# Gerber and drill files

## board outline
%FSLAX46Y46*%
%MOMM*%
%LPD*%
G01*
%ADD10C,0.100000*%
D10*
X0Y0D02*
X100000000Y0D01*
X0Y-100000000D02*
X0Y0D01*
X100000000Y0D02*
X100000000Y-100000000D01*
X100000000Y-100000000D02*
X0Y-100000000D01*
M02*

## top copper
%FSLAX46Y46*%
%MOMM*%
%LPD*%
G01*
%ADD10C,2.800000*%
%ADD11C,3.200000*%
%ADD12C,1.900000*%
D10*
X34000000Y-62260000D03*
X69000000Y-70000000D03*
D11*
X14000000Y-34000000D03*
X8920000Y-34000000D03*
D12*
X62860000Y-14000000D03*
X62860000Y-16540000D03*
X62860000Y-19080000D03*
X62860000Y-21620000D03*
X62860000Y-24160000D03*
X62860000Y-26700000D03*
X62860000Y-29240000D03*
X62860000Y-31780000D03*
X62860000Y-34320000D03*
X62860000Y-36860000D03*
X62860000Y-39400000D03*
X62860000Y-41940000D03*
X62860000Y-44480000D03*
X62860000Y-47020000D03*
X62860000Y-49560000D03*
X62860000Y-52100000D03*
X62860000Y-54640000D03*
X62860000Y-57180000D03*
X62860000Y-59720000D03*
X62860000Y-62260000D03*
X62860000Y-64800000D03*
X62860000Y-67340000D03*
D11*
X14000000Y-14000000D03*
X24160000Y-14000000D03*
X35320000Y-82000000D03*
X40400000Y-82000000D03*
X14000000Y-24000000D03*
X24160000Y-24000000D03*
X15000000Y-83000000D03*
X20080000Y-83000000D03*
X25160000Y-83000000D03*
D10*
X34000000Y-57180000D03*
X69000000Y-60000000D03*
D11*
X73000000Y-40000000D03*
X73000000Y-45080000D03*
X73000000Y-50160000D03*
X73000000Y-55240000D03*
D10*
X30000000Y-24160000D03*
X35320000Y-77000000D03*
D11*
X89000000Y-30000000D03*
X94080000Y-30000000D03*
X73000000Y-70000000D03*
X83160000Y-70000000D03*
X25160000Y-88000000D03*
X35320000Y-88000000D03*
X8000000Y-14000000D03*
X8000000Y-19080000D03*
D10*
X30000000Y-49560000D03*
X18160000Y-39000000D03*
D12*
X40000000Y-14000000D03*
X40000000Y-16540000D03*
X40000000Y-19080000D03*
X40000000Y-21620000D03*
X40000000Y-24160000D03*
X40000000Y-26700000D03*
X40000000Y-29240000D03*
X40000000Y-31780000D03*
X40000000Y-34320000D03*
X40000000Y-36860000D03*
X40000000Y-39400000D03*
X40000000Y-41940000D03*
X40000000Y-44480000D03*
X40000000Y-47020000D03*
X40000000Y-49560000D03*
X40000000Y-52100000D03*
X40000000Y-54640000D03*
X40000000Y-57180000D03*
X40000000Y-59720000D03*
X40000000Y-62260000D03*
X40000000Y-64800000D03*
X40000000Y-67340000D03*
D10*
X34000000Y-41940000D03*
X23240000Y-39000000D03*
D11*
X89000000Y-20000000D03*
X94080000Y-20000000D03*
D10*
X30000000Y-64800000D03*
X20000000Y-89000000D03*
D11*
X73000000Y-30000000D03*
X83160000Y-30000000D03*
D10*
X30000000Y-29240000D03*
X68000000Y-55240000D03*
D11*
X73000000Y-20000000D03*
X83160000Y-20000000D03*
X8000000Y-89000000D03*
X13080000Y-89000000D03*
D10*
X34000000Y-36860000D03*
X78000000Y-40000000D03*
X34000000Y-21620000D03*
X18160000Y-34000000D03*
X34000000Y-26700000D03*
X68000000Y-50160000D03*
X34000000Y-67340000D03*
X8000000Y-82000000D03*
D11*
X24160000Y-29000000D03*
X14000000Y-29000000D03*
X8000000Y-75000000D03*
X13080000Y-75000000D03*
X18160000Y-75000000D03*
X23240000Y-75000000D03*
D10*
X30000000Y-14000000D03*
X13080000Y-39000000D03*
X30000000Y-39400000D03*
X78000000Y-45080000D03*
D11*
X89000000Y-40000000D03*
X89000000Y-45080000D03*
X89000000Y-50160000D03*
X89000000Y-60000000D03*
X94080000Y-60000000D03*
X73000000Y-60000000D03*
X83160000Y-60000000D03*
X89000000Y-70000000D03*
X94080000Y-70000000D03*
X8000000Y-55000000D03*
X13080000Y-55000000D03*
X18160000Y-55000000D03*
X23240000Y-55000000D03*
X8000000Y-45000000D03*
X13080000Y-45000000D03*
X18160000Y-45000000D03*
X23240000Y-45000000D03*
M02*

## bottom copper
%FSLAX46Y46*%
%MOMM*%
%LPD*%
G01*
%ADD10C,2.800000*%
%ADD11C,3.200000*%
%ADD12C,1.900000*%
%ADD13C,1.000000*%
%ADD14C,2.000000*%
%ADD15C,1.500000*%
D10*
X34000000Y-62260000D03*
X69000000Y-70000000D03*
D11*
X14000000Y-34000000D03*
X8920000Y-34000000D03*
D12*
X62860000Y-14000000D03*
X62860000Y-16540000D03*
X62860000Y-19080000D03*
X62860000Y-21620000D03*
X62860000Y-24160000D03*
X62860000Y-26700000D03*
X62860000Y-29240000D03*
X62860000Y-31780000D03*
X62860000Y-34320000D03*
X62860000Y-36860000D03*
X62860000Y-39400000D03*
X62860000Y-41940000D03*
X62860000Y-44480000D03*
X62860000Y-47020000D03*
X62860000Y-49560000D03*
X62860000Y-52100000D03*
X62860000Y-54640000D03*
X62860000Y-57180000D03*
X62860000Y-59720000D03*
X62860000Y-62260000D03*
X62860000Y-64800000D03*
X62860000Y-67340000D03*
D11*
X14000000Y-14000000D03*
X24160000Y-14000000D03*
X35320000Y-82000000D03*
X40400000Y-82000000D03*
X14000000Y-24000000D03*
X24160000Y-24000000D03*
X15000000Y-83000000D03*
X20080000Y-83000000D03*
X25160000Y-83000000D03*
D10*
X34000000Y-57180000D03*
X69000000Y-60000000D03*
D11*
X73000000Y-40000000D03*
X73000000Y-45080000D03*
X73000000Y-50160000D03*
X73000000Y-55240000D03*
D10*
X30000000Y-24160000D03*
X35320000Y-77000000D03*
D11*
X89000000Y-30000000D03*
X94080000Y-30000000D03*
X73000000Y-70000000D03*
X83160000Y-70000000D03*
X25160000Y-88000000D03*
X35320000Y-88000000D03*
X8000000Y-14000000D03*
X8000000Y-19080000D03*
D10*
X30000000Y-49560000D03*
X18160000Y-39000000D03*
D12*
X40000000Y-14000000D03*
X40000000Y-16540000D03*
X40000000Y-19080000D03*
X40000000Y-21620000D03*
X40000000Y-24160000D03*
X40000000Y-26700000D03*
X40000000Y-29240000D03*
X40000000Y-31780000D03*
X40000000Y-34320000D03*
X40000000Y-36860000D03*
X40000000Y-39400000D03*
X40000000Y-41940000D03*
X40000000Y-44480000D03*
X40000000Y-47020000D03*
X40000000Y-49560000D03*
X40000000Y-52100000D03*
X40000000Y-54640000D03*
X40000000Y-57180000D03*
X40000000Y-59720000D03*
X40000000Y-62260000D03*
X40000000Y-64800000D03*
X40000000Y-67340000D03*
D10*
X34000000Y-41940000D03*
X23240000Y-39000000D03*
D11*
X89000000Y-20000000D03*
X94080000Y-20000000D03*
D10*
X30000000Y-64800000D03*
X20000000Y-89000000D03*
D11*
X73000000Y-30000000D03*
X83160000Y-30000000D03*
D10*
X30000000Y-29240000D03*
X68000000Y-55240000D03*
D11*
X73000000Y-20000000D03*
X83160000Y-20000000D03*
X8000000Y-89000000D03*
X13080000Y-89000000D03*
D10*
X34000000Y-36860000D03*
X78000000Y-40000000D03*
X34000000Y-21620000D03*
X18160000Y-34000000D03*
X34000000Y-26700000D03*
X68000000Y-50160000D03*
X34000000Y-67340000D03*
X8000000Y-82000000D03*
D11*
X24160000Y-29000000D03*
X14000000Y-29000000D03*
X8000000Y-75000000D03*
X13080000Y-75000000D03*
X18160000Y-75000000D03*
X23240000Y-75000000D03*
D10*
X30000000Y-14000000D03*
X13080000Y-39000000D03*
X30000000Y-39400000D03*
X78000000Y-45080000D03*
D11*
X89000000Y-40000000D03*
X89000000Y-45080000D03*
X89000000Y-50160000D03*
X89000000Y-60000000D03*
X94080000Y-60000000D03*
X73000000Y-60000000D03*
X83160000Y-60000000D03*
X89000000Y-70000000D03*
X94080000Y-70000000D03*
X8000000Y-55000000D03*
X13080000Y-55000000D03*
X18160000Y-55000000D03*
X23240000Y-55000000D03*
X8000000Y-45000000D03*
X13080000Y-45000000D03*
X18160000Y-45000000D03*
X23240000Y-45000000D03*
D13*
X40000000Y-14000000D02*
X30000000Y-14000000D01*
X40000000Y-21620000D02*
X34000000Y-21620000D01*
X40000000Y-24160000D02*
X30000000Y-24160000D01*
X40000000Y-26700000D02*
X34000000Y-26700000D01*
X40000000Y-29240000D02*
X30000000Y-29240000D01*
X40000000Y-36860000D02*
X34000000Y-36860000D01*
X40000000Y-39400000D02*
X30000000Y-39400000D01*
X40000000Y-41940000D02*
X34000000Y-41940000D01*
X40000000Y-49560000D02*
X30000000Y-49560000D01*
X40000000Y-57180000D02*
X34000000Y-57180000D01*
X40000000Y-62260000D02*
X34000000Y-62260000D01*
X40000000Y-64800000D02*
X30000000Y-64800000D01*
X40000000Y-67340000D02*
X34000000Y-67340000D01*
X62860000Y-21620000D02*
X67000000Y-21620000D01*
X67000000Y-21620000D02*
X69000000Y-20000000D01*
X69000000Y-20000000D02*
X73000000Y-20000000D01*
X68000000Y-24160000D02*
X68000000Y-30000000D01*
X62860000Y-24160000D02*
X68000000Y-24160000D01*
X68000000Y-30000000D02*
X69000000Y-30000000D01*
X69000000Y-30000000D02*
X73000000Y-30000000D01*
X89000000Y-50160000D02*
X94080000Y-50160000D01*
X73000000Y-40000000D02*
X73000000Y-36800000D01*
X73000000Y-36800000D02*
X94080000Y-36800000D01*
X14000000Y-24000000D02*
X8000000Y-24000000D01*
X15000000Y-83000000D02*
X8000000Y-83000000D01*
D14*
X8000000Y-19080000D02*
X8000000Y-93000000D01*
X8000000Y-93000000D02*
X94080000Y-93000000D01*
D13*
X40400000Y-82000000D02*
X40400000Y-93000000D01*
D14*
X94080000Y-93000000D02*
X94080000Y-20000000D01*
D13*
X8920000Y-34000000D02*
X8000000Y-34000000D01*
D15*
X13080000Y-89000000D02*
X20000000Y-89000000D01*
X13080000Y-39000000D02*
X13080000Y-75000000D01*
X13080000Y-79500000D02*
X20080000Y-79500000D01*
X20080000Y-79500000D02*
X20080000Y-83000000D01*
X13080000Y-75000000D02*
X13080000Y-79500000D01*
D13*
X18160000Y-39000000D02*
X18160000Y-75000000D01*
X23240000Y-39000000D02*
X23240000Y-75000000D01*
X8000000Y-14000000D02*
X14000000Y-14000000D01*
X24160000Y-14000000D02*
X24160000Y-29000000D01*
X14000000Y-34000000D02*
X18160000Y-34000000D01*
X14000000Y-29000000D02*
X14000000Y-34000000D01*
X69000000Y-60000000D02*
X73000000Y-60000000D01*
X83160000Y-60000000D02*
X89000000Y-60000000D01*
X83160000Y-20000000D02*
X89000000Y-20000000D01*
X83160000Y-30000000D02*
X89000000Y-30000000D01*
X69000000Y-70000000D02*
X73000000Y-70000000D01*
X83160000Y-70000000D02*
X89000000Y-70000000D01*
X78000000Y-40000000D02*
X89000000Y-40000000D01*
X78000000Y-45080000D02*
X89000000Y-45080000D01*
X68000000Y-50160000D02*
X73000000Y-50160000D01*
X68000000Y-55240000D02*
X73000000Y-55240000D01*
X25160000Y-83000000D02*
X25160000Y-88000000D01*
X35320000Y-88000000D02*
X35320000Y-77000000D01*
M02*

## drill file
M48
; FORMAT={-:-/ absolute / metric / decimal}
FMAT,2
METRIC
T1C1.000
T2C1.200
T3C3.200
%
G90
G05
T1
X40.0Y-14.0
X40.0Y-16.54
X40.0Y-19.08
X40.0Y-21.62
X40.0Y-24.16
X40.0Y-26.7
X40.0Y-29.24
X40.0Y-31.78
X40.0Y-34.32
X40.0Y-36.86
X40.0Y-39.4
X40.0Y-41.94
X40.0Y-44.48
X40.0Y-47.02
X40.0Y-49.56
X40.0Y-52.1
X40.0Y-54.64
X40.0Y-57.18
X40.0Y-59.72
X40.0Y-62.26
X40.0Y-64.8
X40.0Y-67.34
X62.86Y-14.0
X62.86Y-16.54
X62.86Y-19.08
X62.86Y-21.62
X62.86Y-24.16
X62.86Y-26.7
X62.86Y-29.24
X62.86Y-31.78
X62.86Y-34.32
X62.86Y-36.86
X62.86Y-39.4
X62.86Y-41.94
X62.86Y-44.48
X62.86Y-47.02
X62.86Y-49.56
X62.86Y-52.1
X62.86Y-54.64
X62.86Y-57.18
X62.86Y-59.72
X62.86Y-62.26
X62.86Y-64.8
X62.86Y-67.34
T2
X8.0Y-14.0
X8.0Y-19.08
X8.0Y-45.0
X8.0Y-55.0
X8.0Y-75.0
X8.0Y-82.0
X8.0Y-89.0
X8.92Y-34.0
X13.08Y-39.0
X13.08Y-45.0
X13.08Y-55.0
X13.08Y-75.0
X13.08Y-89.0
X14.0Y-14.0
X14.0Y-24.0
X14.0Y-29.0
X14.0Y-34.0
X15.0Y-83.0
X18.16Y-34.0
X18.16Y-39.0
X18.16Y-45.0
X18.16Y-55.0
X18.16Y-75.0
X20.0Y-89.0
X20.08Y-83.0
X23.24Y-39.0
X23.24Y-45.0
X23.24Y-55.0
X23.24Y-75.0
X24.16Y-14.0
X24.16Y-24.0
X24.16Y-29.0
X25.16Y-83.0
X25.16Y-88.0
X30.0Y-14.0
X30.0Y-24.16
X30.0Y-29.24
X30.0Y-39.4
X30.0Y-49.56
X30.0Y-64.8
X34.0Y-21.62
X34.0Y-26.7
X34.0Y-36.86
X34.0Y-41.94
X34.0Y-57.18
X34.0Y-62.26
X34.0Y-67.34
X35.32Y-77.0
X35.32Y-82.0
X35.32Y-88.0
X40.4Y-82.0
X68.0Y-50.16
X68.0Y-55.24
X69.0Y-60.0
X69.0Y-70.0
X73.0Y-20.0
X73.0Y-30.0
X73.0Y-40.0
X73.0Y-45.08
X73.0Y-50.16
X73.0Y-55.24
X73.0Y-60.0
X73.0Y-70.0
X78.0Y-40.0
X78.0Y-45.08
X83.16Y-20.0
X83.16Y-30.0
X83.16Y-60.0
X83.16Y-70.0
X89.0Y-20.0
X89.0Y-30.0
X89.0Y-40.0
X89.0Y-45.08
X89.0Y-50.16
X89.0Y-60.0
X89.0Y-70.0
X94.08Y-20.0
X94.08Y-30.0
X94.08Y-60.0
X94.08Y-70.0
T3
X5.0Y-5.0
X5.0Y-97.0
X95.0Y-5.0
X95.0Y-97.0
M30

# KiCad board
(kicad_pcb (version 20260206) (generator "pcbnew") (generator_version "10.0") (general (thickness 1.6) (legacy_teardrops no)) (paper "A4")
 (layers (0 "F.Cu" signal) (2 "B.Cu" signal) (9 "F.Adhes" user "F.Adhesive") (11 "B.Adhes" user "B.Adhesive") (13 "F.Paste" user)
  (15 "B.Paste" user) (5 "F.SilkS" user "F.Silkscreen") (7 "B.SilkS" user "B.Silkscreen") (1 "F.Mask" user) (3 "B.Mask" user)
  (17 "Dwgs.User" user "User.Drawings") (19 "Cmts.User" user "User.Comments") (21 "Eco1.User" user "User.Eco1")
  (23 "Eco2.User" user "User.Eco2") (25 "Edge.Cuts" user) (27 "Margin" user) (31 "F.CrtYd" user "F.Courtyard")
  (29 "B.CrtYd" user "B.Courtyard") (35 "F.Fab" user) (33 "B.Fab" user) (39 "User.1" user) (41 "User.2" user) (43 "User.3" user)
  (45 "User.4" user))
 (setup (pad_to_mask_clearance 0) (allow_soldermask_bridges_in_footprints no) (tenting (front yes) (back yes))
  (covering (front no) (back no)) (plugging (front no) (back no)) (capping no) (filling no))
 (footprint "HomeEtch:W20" (layer "F.Cu") (at 34 62.26)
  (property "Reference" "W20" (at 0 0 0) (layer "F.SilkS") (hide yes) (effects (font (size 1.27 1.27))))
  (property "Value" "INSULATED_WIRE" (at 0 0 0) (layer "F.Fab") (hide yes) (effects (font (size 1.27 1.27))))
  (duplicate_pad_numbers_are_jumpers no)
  (pad "1" thru_hole circle (at 0 0) (size 2.8 2.8) (drill 1.2) (layers "*.Cu" "*.Mask") (remove_unused_layers no) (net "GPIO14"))
  (pad "2" thru_hole circle (at 35 7.74) (size 2.8 2.8) (drill 1.2) (layers "*.Cu" "*.Mask") (remove_unused_layers no) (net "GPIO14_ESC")))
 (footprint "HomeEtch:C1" (layer "F.Cu") (at 14 34)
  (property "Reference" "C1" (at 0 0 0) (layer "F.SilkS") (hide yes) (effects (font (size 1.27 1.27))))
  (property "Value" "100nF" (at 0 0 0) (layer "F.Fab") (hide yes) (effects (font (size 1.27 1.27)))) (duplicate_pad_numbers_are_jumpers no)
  (pad "1" thru_hole circle (at 0 0) (size 3.2 3.2) (drill 1.2) (layers "*.Cu" "*.Mask") (remove_unused_layers no) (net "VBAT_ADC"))
  (pad "2" thru_hole circle (at -5.08 0) (size 3.2 3.2) (drill 1.2) (layers "*.Cu" "*.Mask") (remove_unused_layers no) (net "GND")))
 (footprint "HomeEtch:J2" (layer "F.Cu") (at 62.86 14)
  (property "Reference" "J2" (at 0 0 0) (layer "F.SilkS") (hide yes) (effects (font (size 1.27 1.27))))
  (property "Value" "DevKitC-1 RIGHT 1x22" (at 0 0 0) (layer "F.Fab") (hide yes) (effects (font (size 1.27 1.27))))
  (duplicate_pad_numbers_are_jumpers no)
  (pad "1" thru_hole circle (at 0 0) (size 1.9 1.9) (drill 1) (layers "*.Cu" "*.Mask") (remove_unused_layers no)
   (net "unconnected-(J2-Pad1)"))
  (pad "2" thru_hole circle (at 0 2.54) (size 1.9 1.9) (drill 1) (layers "*.Cu" "*.Mask") (remove_unused_layers no)
   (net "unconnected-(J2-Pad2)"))
  (pad "3" thru_hole circle (at 0 5.08) (size 1.9 1.9) (drill 1) (layers "*.Cu" "*.Mask") (remove_unused_layers no)
   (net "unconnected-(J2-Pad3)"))
  (pad "4" thru_hole circle (at 0 7.62) (size 1.9 1.9) (drill 1) (layers "*.Cu" "*.Mask") (remove_unused_layers no) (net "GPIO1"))
  (pad "5" thru_hole circle (at 0 10.16) (size 1.9 1.9) (drill 1) (layers "*.Cu" "*.Mask") (remove_unused_layers no) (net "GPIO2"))
  (pad "6" thru_hole circle (at 0 12.7) (size 1.9 1.9) (drill 1) (layers "*.Cu" "*.Mask") (remove_unused_layers no)
   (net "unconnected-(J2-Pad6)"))
  (pad "7" thru_hole circle (at 0 15.24) (size 1.9 1.9) (drill 1) (layers "*.Cu" "*.Mask") (remove_unused_layers no)
   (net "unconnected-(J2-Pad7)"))
  (pad "8" thru_hole circle (at 0 17.78) (size 1.9 1.9) (drill 1) (layers "*.Cu" "*.Mask") (remove_unused_layers no)
   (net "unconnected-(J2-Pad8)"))
  (pad "9" thru_hole circle (at 0 20.32) (size 1.9 1.9) (drill 1) (layers "*.Cu" "*.Mask") (remove_unused_layers no)
   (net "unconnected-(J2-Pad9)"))
  (pad "10" thru_hole circle (at 0 22.86) (size 1.9 1.9) (drill 1) (layers "*.Cu" "*.Mask") (remove_unused_layers no)
   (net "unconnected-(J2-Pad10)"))
  (pad "11" thru_hole circle (at 0 25.4) (size 1.9 1.9) (drill 1) (layers "*.Cu" "*.Mask") (remove_unused_layers no)
   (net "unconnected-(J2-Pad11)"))
  (pad "12" thru_hole circle (at 0 27.94) (size 1.9 1.9) (drill 1) (layers "*.Cu" "*.Mask") (remove_unused_layers no)
   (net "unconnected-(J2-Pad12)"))
  (pad "13" thru_hole circle (at 0 30.48) (size 1.9 1.9) (drill 1) (layers "*.Cu" "*.Mask") (remove_unused_layers no)
   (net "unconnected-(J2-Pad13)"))
  (pad "14" thru_hole circle (at 0 33.02) (size 1.9 1.9) (drill 1) (layers "*.Cu" "*.Mask") (remove_unused_layers no)
   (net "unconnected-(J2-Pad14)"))
  (pad "15" thru_hole circle (at 0 35.56) (size 1.9 1.9) (drill 1) (layers "*.Cu" "*.Mask") (remove_unused_layers no)
   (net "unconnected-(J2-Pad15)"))
  (pad "16" thru_hole circle (at 0 38.1) (size 1.9 1.9) (drill 1) (layers "*.Cu" "*.Mask") (remove_unused_layers no)
   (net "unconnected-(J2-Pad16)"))
  (pad "17" thru_hole circle (at 0 40.64) (size 1.9 1.9) (drill 1) (layers "*.Cu" "*.Mask") (remove_unused_layers no)
   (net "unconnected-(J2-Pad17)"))
  (pad "18" thru_hole circle (at 0 43.18) (size 1.9 1.9) (drill 1) (layers "*.Cu" "*.Mask") (remove_unused_layers no)
   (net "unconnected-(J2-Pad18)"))
  (pad "19" thru_hole circle (at 0 45.72) (size 1.9 1.9) (drill 1) (layers "*.Cu" "*.Mask") (remove_unused_layers no)
   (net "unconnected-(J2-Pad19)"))
  (pad "20" thru_hole circle (at 0 48.26) (size 1.9 1.9) (drill 1) (layers "*.Cu" "*.Mask") (remove_unused_layers no)
   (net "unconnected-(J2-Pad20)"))
  (pad "21" thru_hole circle (at 0 50.8) (size 1.9 1.9) (drill 1) (layers "*.Cu" "*.Mask") (remove_unused_layers no)
   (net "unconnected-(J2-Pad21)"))
  (pad "22" thru_hole circle (at 0 53.34) (size 1.9 1.9) (drill 1) (layers "*.Cu" "*.Mask") (remove_unused_layers no)
   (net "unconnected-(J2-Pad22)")))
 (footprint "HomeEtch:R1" (layer "F.Cu") (at 14 14)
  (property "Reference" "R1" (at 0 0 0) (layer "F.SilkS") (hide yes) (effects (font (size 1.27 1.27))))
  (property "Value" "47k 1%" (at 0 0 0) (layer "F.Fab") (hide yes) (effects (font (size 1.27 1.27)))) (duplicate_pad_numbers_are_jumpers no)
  (pad "1" thru_hole circle (at 0 0) (size 3.2 3.2) (drill 1.2) (layers "*.Cu" "*.Mask") (remove_unused_layers no) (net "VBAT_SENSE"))
  (pad "2" thru_hole circle (at 10.16 0) (size 3.2 3.2) (drill 1.2) (layers "*.Cu" "*.Mask") (remove_unused_layers no) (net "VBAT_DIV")))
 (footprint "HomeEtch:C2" (layer "F.Cu") (at 35.32 82)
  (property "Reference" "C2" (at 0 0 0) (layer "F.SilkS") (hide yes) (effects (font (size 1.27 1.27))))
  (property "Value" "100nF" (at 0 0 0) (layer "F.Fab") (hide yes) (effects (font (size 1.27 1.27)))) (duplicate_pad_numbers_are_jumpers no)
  (pad "1" thru_hole circle (at 0 0) (size 3.2 3.2) (drill 1.2) (layers "*.Cu" "*.Mask") (remove_unused_layers no) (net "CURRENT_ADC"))
  (pad "2" thru_hole circle (at 5.08 0) (size 3.2 3.2) (drill 1.2) (layers "*.Cu" "*.Mask") (remove_unused_layers no) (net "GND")))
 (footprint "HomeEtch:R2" (layer "F.Cu") (at 14 24)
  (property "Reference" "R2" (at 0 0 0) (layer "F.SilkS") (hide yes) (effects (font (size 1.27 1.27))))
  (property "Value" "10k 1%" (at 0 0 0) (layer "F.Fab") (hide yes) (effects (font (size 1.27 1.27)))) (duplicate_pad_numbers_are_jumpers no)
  (pad "1" thru_hole circle (at 0 0) (size 3.2 3.2) (drill 1.2) (layers "*.Cu" "*.Mask") (remove_unused_layers no) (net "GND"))
  (pad "2" thru_hole circle (at 10.16 0) (size 3.2 3.2) (drill 1.2) (layers "*.Cu" "*.Mask") (remove_unused_layers no) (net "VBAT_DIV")))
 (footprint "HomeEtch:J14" (layer "F.Cu") (at 15 83)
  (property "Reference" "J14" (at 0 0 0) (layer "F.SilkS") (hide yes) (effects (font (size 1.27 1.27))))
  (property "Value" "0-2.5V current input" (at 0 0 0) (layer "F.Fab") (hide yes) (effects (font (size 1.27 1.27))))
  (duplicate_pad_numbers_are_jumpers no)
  (pad "1" thru_hole circle (at 0 0) (size 3.2 3.2) (drill 1.2) (layers "*.Cu" "*.Mask") (remove_unused_layers no) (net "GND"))
  (pad "2" thru_hole circle (at 5.08 0) (size 3.2 3.2) (drill 1.2) (layers "*.Cu" "*.Mask") (remove_unused_layers no) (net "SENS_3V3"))
  (pad "3" thru_hole circle (at 10.16 0) (size 3.2 3.2) (drill 1.2) (layers "*.Cu" "*.Mask") (remove_unused_layers no) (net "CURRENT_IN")))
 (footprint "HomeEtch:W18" (layer "F.Cu") (at 34 57.18)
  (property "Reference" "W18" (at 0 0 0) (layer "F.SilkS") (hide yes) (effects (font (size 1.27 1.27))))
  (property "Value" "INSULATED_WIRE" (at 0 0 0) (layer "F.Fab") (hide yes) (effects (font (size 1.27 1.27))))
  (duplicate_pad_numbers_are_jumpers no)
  (pad "1" thru_hole circle (at 0 0) (size 2.8 2.8) (drill 1.2) (layers "*.Cu" "*.Mask") (remove_unused_layers no) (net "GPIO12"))
  (pad "2" thru_hole circle (at 35 2.82) (size 2.8 2.8) (drill 1.2) (layers "*.Cu" "*.Mask") (remove_unused_layers no) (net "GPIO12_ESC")))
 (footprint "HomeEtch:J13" (layer "F.Cu") (at 73 40)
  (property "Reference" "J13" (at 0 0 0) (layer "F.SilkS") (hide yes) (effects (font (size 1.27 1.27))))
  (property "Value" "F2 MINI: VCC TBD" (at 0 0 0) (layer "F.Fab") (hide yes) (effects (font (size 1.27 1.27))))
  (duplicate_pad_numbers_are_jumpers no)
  (pad "1" thru_hole circle (at 0 0) (size 3.2 3.2) (drill 1.2) (layers "*.Cu" "*.Mask") (remove_unused_layers no) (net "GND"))
  (pad "2" thru_hole circle (at 0 5.08) (size 3.2 3.2) (drill 1.2) (layers "*.Cu" "*.Mask") (remove_unused_layers no)
   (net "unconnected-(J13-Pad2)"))
  (pad "3" thru_hole circle (at 0 10.16) (size 3.2 3.2) (drill 1.2) (layers "*.Cu" "*.Mask") (remove_unused_layers no) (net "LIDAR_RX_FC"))
  (pad "4" thru_hole circle (at 0 15.24) (size 3.2 3.2) (drill 1.2) (layers "*.Cu" "*.Mask") (remove_unused_layers no) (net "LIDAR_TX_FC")))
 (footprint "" (layer "F.Cu") (at 5 5)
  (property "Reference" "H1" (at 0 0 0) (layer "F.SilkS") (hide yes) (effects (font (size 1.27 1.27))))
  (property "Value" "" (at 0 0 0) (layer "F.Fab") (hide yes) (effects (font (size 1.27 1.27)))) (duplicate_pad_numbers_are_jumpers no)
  (pad "" np_thru_hole circle (at 0 0) (size 3.2 3.2) (drill 3.2) (layers "*.Cu" "*.Mask")))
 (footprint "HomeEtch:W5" (layer "F.Cu") (at 30 24.16)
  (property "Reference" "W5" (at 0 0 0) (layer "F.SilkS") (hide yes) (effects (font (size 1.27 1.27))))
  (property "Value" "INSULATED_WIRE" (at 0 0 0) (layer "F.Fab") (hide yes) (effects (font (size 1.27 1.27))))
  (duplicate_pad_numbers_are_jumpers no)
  (pad "1" thru_hole circle (at 0 0) (size 2.8 2.8) (drill 1.2) (layers "*.Cu" "*.Mask") (remove_unused_layers no) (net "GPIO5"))
  (pad "2" thru_hole circle (at 5.32 52.84) (size 2.8 2.8) (drill 1.2) (layers "*.Cu" "*.Mask") (remove_unused_layers no)
   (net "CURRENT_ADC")))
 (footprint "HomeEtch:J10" (layer "F.Cu") (at 89 30)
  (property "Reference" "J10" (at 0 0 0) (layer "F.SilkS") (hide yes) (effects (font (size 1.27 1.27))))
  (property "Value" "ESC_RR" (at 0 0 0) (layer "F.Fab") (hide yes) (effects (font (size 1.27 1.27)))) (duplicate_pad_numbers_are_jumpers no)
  (pad "1" thru_hole circle (at 0 0) (size 3.2 3.2) (drill 1.2) (layers "*.Cu" "*.Mask") (remove_unused_layers no) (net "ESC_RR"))
  (pad "2" thru_hole circle (at 5.08 0) (size 3.2 3.2) (drill 1.2) (layers "*.Cu" "*.Mask") (remove_unused_layers no) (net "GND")))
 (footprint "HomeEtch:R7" (layer "F.Cu") (at 73 70)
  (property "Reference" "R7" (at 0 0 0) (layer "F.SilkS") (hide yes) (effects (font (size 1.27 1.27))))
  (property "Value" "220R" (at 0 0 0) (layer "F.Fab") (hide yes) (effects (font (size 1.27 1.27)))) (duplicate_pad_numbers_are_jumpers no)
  (pad "1" thru_hole circle (at 0 0) (size 3.2 3.2) (drill 1.2) (layers "*.Cu" "*.Mask") (remove_unused_layers no) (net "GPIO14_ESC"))
  (pad "2" thru_hole circle (at 10.16 0) (size 3.2 3.2) (drill 1.2) (layers "*.Cu" "*.Mask") (remove_unused_layers no) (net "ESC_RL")))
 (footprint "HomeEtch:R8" (layer "F.Cu") (at 25.16 88)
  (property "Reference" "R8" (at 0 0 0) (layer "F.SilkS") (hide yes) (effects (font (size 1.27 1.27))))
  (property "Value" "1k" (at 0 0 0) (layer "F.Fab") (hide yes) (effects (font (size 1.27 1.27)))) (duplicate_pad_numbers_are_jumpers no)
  (pad "1" thru_hole circle (at 0 0) (size 3.2 3.2) (drill 1.2) (layers "*.Cu" "*.Mask") (remove_unused_layers no) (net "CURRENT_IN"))
  (pad "2" thru_hole circle (at 10.16 0) (size 3.2 3.2) (drill 1.2) (layers "*.Cu" "*.Mask") (remove_unused_layers no) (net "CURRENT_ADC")))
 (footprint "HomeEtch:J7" (layer "F.Cu") (at 8 14)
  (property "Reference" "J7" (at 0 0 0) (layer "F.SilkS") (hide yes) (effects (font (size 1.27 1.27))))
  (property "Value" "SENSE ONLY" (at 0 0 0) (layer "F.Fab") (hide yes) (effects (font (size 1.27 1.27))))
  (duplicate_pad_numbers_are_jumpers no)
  (pad "1" thru_hole circle (at 0 0) (size 3.2 3.2) (drill 1.2) (layers "*.Cu" "*.Mask") (remove_unused_layers no) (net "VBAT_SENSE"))
  (pad "2" thru_hole circle (at 0 5.08) (size 3.2 3.2) (drill 1.2) (layers "*.Cu" "*.Mask") (remove_unused_layers no) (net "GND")))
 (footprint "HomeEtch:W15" (layer "F.Cu") (at 30 49.56)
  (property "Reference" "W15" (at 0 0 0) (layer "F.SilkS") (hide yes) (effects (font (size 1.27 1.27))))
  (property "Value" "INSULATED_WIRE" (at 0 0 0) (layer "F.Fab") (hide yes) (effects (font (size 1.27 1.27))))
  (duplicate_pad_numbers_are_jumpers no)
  (pad "1" thru_hole circle (at 0 0) (size 2.8 2.8) (drill 1.2) (layers "*.Cu" "*.Mask") (remove_unused_layers no) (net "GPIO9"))
  (pad "2" thru_hole circle (at -11.84 -10.56) (size 2.8 2.8) (drill 1.2) (layers "*.Cu" "*.Mask") (remove_unused_layers no) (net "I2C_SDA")))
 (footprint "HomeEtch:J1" (layer "F.Cu") (at 40 14)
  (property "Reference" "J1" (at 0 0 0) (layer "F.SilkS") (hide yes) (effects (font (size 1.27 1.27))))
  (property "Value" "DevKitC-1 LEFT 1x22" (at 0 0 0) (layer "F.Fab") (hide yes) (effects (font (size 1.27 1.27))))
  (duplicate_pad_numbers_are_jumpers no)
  (pad "1" thru_hole circle (at 0 0) (size 1.9 1.9) (drill 1) (layers "*.Cu" "*.Mask") (remove_unused_layers no) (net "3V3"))
  (pad "2" thru_hole circle (at 0 2.54) (size 1.9 1.9) (drill 1) (layers "*.Cu" "*.Mask") (remove_unused_layers no)
   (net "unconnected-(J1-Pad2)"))
  (pad "3" thru_hole circle (at 0 5.08) (size 1.9 1.9) (drill 1) (layers "*.Cu" "*.Mask") (remove_unused_layers no)
   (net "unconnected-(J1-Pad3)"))
  (pad "4" thru_hole circle (at 0 7.62) (size 1.9 1.9) (drill 1) (layers "*.Cu" "*.Mask") (remove_unused_layers no) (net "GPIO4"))
  (pad "5" thru_hole circle (at 0 10.16) (size 1.9 1.9) (drill 1) (layers "*.Cu" "*.Mask") (remove_unused_layers no) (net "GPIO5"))
  (pad "6" thru_hole circle (at 0 12.7) (size 1.9 1.9) (drill 1) (layers "*.Cu" "*.Mask") (remove_unused_layers no) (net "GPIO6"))
  (pad "7" thru_hole circle (at 0 15.24) (size 1.9 1.9) (drill 1) (layers "*.Cu" "*.Mask") (remove_unused_layers no) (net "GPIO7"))
  (pad "8" thru_hole circle (at 0 17.78) (size 1.9 1.9) (drill 1) (layers "*.Cu" "*.Mask") (remove_unused_layers no)
   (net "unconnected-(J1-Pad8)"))
  (pad "9" thru_hole circle (at 0 20.32) (size 1.9 1.9) (drill 1) (layers "*.Cu" "*.Mask") (remove_unused_layers no)
   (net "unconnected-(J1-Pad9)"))
  (pad "10" thru_hole circle (at 0 22.86) (size 1.9 1.9) (drill 1) (layers "*.Cu" "*.Mask") (remove_unused_layers no) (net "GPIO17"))
  (pad "11" thru_hole circle (at 0 25.4) (size 1.9 1.9) (drill 1) (layers "*.Cu" "*.Mask") (remove_unused_layers no) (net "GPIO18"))
  (pad "12" thru_hole circle (at 0 27.94) (size 1.9 1.9) (drill 1) (layers "*.Cu" "*.Mask") (remove_unused_layers no) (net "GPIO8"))
  (pad "13" thru_hole circle (at 0 30.48) (size 1.9 1.9) (drill 1) (layers "*.Cu" "*.Mask") (remove_unused_layers no)
   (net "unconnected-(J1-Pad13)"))
  (pad "14" thru_hole circle (at 0 33.02) (size 1.9 1.9) (drill 1) (layers "*.Cu" "*.Mask") (remove_unused_layers no)
   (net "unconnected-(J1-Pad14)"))
  (pad "15" thru_hole circle (at 0 35.56) (size 1.9 1.9) (drill 1) (layers "*.Cu" "*.Mask") (remove_unused_layers no) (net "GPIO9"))
  (pad "16" thru_hole circle (at 0 38.1) (size 1.9 1.9) (drill 1) (layers "*.Cu" "*.Mask") (remove_unused_layers no)
   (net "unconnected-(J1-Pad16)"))
  (pad "17" thru_hole circle (at 0 40.64) (size 1.9 1.9) (drill 1) (layers "*.Cu" "*.Mask") (remove_unused_layers no)
   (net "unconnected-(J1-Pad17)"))
  (pad "18" thru_hole circle (at 0 43.18) (size 1.9 1.9) (drill 1) (layers "*.Cu" "*.Mask") (remove_unused_layers no) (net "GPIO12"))
  (pad "19" thru_hole circle (at 0 45.72) (size 1.9 1.9) (drill 1) (layers "*.Cu" "*.Mask") (remove_unused_layers no)
   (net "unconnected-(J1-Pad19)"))
  (pad "20" thru_hole circle (at 0 48.26) (size 1.9 1.9) (drill 1) (layers "*.Cu" "*.Mask") (remove_unused_layers no) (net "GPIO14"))
  (pad "21" thru_hole circle (at 0 50.8) (size 1.9 1.9) (drill 1) (layers "*.Cu" "*.Mask") (remove_unused_layers no) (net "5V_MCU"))
  (pad "22" thru_hole circle (at 0 53.34) (size 1.9 1.9) (drill 1) (layers "*.Cu" "*.Mask") (remove_unused_layers no) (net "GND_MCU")))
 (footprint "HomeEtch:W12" (layer "F.Cu") (at 34 41.94)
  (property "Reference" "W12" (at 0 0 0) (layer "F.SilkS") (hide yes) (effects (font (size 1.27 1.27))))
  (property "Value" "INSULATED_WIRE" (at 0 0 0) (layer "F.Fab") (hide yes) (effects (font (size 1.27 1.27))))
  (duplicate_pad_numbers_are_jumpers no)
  (pad "1" thru_hole circle (at 0 0) (size 2.8 2.8) (drill 1.2) (layers "*.Cu" "*.Mask") (remove_unused_layers no) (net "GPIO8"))
  (pad "2" thru_hole circle (at -10.76 -2.94) (size 2.8 2.8) (drill 1.2) (layers "*.Cu" "*.Mask") (remove_unused_layers no) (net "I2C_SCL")))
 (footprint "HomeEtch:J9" (layer "F.Cu") (at 89 20)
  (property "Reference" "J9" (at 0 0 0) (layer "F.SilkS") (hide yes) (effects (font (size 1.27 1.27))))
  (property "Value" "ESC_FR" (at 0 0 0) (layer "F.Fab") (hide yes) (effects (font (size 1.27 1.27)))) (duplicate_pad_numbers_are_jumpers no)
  (pad "1" thru_hole circle (at 0 0) (size 3.2 3.2) (drill 1.2) (layers "*.Cu" "*.Mask") (remove_unused_layers no) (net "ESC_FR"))
  (pad "2" thru_hole circle (at 5.08 0) (size 3.2 3.2) (drill 1.2) (layers "*.Cu" "*.Mask") (remove_unused_layers no) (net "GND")))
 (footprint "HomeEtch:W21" (layer "F.Cu") (at 30 64.8)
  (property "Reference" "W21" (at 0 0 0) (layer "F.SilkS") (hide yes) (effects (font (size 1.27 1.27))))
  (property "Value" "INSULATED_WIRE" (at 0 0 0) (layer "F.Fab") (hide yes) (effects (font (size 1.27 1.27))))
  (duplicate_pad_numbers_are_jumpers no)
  (pad "1" thru_hole circle (at 0 0) (size 2.8 2.8) (drill 1.2) (layers "*.Cu" "*.Mask") (remove_unused_layers no) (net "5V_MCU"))
  (pad "2" thru_hole circle (at -10 24.2) (size 2.8 2.8) (drill 1.2) (layers "*.Cu" "*.Mask") (remove_unused_layers no) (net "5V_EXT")))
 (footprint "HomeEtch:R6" (layer "F.Cu") (at 73 30)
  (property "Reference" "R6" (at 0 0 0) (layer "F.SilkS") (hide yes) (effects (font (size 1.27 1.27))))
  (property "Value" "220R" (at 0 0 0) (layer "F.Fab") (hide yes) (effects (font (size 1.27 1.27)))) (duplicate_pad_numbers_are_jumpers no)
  (pad "1" thru_hole circle (at 0 0) (size 3.2 3.2) (drill 1.2) (layers "*.Cu" "*.Mask") (remove_unused_layers no) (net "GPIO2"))
  (pad "2" thru_hole circle (at 10.16 0) (size 3.2 3.2) (drill 1.2) (layers "*.Cu" "*.Mask") (remove_unused_layers no) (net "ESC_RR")))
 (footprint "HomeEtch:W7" (layer "F.Cu") (at 30 29.24)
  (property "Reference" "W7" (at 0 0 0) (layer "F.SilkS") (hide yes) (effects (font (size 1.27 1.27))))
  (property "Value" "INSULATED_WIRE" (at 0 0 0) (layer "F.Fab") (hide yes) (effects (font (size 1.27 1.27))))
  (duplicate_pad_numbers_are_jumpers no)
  (pad "1" thru_hole circle (at 0 0) (size 2.8 2.8) (drill 1.2) (layers "*.Cu" "*.Mask") (remove_unused_layers no) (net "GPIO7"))
  (pad "2" thru_hole circle (at 38 26) (size 2.8 2.8) (drill 1.2) (layers "*.Cu" "*.Mask") (remove_unused_layers no) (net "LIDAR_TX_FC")))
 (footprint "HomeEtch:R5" (layer "F.Cu") (at 73 20)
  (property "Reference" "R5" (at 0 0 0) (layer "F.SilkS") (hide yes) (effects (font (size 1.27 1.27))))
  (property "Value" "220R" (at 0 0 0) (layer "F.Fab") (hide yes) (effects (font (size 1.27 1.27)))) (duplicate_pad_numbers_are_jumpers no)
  (pad "1" thru_hole circle (at 0 0) (size 3.2 3.2) (drill 1.2) (layers "*.Cu" "*.Mask") (remove_unused_layers no) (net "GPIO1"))
  (pad "2" thru_hole circle (at 10.16 0) (size 3.2 3.2) (drill 1.2) (layers "*.Cu" "*.Mask") (remove_unused_layers no) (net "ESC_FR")))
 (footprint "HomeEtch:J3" (layer "F.Cu") (at 8 89)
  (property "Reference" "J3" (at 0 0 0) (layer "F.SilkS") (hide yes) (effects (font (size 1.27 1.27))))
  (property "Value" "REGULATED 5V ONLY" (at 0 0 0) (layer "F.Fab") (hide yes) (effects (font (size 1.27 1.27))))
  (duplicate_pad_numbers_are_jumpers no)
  (pad "1" thru_hole circle (at 0 0) (size 3.2 3.2) (drill 1.2) (layers "*.Cu" "*.Mask") (remove_unused_layers no) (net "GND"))
  (pad "2" thru_hole circle (at 5.08 0) (size 3.2 3.2) (drill 1.2) (layers "*.Cu" "*.Mask") (remove_unused_layers no) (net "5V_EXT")))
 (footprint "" (layer "F.Cu") (at 5 97)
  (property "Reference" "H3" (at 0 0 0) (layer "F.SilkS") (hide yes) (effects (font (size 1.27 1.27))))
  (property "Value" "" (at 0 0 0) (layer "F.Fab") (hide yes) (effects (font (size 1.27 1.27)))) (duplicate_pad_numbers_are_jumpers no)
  (pad "" np_thru_hole circle (at 0 0) (size 3.2 3.2) (drill 3.2) (layers "*.Cu" "*.Mask")))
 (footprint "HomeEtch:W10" (layer "F.Cu") (at 34 36.86)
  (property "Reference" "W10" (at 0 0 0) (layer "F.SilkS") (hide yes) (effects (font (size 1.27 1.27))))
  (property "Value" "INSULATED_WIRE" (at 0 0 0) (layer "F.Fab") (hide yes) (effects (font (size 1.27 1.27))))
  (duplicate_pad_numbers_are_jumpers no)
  (pad "1" thru_hole circle (at 0 0) (size 2.8 2.8) (drill 1.2) (layers "*.Cu" "*.Mask") (remove_unused_layers no) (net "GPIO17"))
  (pad "2" thru_hole circle (at 44 3.14) (size 2.8 2.8) (drill 1.2) (layers "*.Cu" "*.Mask") (remove_unused_layers no) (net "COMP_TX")))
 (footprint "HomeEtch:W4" (layer "F.Cu") (at 34 21.62)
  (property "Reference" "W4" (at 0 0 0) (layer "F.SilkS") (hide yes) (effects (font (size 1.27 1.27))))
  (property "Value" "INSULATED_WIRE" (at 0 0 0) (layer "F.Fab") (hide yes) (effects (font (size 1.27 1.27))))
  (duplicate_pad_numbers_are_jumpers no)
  (pad "1" thru_hole circle (at 0 0) (size 2.8 2.8) (drill 1.2) (layers "*.Cu" "*.Mask") (remove_unused_layers no) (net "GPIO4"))
  (pad "2" thru_hole circle (at -15.84 12.38) (size 2.8 2.8) (drill 1.2) (layers "*.Cu" "*.Mask") (remove_unused_layers no) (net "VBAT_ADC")))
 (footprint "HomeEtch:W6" (layer "F.Cu") (at 34 26.7)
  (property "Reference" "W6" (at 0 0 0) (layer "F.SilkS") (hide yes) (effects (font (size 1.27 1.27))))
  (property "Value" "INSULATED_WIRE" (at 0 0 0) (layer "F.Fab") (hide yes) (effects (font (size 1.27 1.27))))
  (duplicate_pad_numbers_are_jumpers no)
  (pad "1" thru_hole circle (at 0 0) (size 2.8 2.8) (drill 1.2) (layers "*.Cu" "*.Mask") (remove_unused_layers no) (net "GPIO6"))
  (pad "2" thru_hole circle (at 34 23.46) (size 2.8 2.8) (drill 1.2) (layers "*.Cu" "*.Mask") (remove_unused_layers no) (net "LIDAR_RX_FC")))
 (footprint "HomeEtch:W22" (layer "F.Cu") (at 34 67.34)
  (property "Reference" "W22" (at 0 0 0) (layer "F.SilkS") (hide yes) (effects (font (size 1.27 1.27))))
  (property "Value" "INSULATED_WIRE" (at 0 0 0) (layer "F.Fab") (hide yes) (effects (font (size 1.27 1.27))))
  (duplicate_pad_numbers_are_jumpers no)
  (pad "1" thru_hole circle (at 0 0) (size 2.8 2.8) (drill 1.2) (layers "*.Cu" "*.Mask") (remove_unused_layers no) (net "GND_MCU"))
  (pad "2" thru_hole circle (at -26 14.66) (size 2.8 2.8) (drill 1.2) (layers "*.Cu" "*.Mask") (remove_unused_layers no) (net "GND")))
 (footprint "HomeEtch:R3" (layer "F.Cu") (at 24.16 29)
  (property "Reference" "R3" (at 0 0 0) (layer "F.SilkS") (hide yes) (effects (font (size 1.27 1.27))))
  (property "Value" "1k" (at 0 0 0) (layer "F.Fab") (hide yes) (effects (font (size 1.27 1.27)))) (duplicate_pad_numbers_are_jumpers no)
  (pad "1" thru_hole circle (at 0 0) (size 3.2 3.2) (drill 1.2) (layers "*.Cu" "*.Mask") (remove_unused_layers no) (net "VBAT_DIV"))
  (pad "2" thru_hole circle (at -10.16 0) (size 3.2 3.2) (drill 1.2) (layers "*.Cu" "*.Mask") (remove_unused_layers no) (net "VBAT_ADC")))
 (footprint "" (layer "F.Cu") (at 95 5)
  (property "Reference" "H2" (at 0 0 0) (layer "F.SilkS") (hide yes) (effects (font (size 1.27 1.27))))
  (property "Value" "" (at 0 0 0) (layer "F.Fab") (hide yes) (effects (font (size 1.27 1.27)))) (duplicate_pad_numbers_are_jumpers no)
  (pad "" np_thru_hole circle (at 0 0) (size 3.2 3.2) (drill 3.2) (layers "*.Cu" "*.Mask")))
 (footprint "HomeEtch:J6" (layer "F.Cu") (at 8 75)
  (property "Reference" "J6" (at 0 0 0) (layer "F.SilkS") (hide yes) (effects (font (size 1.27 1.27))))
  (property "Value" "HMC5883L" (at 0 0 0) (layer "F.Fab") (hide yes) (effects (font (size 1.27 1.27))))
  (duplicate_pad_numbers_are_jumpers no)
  (pad "1" thru_hole circle (at 0 0) (size 3.2 3.2) (drill 1.2) (layers "*.Cu" "*.Mask") (remove_unused_layers no) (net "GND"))
  (pad "2" thru_hole circle (at 5.08 0) (size 3.2 3.2) (drill 1.2) (layers "*.Cu" "*.Mask") (remove_unused_layers no) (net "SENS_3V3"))
  (pad "3" thru_hole circle (at 10.16 0) (size 3.2 3.2) (drill 1.2) (layers "*.Cu" "*.Mask") (remove_unused_layers no) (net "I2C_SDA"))
  (pad "4" thru_hole circle (at 15.24 0) (size 3.2 3.2) (drill 1.2) (layers "*.Cu" "*.Mask") (remove_unused_layers no) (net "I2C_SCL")))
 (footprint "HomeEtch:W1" (layer "F.Cu") (at 30 14)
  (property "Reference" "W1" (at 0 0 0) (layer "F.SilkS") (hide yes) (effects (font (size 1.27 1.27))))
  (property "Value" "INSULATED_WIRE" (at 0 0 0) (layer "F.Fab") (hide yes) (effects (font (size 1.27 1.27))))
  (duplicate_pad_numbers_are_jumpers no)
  (pad "1" thru_hole circle (at 0 0) (size 2.8 2.8) (drill 1.2) (layers "*.Cu" "*.Mask") (remove_unused_layers no) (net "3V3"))
  (pad "2" thru_hole circle (at -16.92 25) (size 2.8 2.8) (drill 1.2) (layers "*.Cu" "*.Mask") (remove_unused_layers no) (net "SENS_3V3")))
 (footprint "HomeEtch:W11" (layer "F.Cu") (at 30 39.4)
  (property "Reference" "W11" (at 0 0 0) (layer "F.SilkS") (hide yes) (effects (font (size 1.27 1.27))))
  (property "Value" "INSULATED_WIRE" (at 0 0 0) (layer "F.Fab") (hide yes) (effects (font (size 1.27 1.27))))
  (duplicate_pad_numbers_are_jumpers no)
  (pad "1" thru_hole circle (at 0 0) (size 2.8 2.8) (drill 1.2) (layers "*.Cu" "*.Mask") (remove_unused_layers no) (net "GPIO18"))
  (pad "2" thru_hole circle (at 48 5.68) (size 2.8 2.8) (drill 1.2) (layers "*.Cu" "*.Mask") (remove_unused_layers no) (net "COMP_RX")))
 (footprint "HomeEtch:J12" (layer "F.Cu") (at 89 40)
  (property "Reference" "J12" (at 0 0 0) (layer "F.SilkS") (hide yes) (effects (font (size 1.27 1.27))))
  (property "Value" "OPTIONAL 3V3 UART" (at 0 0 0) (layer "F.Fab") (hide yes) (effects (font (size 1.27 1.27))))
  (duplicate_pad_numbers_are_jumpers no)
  (pad "1" thru_hole circle (at 0 0) (size 3.2 3.2) (drill 1.2) (layers "*.Cu" "*.Mask") (remove_unused_layers no) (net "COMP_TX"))
  (pad "2" thru_hole circle (at 0 5.08) (size 3.2 3.2) (drill 1.2) (layers "*.Cu" "*.Mask") (remove_unused_layers no) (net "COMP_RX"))
  (pad "3" thru_hole circle (at 0 10.16) (size 3.2 3.2) (drill 1.2) (layers "*.Cu" "*.Mask") (remove_unused_layers no) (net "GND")))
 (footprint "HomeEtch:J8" (layer "F.Cu") (at 89 60)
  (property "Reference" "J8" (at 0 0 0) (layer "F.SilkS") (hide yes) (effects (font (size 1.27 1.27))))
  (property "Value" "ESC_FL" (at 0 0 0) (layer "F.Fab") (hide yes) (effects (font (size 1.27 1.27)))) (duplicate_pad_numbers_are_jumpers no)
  (pad "1" thru_hole circle (at 0 0) (size 3.2 3.2) (drill 1.2) (layers "*.Cu" "*.Mask") (remove_unused_layers no) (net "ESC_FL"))
  (pad "2" thru_hole circle (at 5.08 0) (size 3.2 3.2) (drill 1.2) (layers "*.Cu" "*.Mask") (remove_unused_layers no) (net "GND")))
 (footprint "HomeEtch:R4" (layer "F.Cu") (at 73 60)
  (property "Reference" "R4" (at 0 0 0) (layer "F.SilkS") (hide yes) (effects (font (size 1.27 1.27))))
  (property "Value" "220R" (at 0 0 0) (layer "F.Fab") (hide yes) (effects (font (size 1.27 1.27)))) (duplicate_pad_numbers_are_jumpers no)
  (pad "1" thru_hole circle (at 0 0) (size 3.2 3.2) (drill 1.2) (layers "*.Cu" "*.Mask") (remove_unused_layers no) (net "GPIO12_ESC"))
  (pad "2" thru_hole circle (at 10.16 0) (size 3.2 3.2) (drill 1.2) (layers "*.Cu" "*.Mask") (remove_unused_layers no) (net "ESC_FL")))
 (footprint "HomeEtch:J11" (layer "F.Cu") (at 89 70)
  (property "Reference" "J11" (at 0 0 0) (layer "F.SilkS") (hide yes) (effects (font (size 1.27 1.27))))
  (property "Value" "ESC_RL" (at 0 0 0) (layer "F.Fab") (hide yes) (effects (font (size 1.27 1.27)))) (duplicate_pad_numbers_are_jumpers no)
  (pad "1" thru_hole circle (at 0 0) (size 3.2 3.2) (drill 1.2) (layers "*.Cu" "*.Mask") (remove_unused_layers no) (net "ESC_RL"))
  (pad "2" thru_hole circle (at 5.08 0) (size 3.2 3.2) (drill 1.2) (layers "*.Cu" "*.Mask") (remove_unused_layers no) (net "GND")))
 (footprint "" (layer "F.Cu") (at 95 97)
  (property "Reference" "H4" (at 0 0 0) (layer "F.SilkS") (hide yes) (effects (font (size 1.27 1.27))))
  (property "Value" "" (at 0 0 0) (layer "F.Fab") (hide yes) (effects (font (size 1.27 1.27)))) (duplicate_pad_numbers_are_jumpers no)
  (pad "" np_thru_hole circle (at 0 0) (size 3.2 3.2) (drill 3.2) (layers "*.Cu" "*.Mask")))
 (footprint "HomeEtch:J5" (layer "F.Cu") (at 8 55)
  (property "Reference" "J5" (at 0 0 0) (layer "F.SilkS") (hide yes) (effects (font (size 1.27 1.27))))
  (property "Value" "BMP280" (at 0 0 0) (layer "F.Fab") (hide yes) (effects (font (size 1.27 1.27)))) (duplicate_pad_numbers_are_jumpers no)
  (pad "1" thru_hole circle (at 0 0) (size 3.2 3.2) (drill 1.2) (layers "*.Cu" "*.Mask") (remove_unused_layers no) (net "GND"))
  (pad "2" thru_hole circle (at 5.08 0) (size 3.2 3.2) (drill 1.2) (layers "*.Cu" "*.Mask") (remove_unused_layers no) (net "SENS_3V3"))
  (pad "3" thru_hole circle (at 10.16 0) (size 3.2 3.2) (drill 1.2) (layers "*.Cu" "*.Mask") (remove_unused_layers no) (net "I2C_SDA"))
  (pad "4" thru_hole circle (at 15.24 0) (size 3.2 3.2) (drill 1.2) (layers "*.Cu" "*.Mask") (remove_unused_layers no) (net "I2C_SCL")))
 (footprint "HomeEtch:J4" (layer "F.Cu") (at 8 45)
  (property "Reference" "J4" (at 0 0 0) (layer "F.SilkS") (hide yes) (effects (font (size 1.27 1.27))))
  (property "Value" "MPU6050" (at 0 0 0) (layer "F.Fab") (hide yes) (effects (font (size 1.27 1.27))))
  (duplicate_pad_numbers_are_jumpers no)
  (pad "1" thru_hole circle (at 0 0) (size 3.2 3.2) (drill 1.2) (layers "*.Cu" "*.Mask") (remove_unused_layers no) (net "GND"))
  (pad "2" thru_hole circle (at 5.08 0) (size 3.2 3.2) (drill 1.2) (layers "*.Cu" "*.Mask") (remove_unused_layers no) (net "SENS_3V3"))
  (pad "3" thru_hole circle (at 10.16 0) (size 3.2 3.2) (drill 1.2) (layers "*.Cu" "*.Mask") (remove_unused_layers no) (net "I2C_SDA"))
  (pad "4" thru_hole circle (at 15.24 0) (size 3.2 3.2) (drill 1.2) (layers "*.Cu" "*.Mask") (remove_unused_layers no) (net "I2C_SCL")))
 (gr_line (start 0 0) (end 100 0) (stroke (width 0.1) (type default)) (layer "Edge.Cuts"))
 (gr_line (start 0 100) (end 0 0) (stroke (width 0.1) (type default)) (layer "Edge.Cuts"))
 (gr_line (start 100 0) (end 100 100) (stroke (width 0.1) (type default)) (layer "Edge.Cuts"))
 (gr_line (start 100 100) (end 0 100) (stroke (width 0.1) (type default)) (layer "Edge.Cuts"))
 (segment (start 40 14) (end 30 14) (width 1) (layer "B.Cu") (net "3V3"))
 (segment (start 40 21.62) (end 34 21.62) (width 1) (layer "B.Cu") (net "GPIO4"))
 (segment (start 40 24.16) (end 30 24.16) (width 1) (layer "B.Cu") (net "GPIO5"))
 (segment (start 40 26.7) (end 34 26.7) (width 1) (layer "B.Cu") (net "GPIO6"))
 (segment (start 40 29.24) (end 30 29.24) (width 1) (layer "B.Cu") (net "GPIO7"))
 (segment (start 40 36.86) (end 34 36.86) (width 1) (layer "B.Cu") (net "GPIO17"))
 (segment (start 40 39.4) (end 30 39.4) (width 1) (layer "B.Cu") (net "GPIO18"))
 (segment (start 40 41.94) (end 34 41.94) (width 1) (layer "B.Cu") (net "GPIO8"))
 (segment (start 40 49.56) (end 30 49.56) (width 1) (layer "B.Cu") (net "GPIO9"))
 (segment (start 40 57.18) (end 34 57.18) (width 1) (layer "B.Cu") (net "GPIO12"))
 (segment (start 40 62.26) (end 34 62.26) (width 1) (layer "B.Cu") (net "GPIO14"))
 (segment (start 40 64.8) (end 30 64.8) (width 1) (layer "B.Cu") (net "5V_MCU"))
 (segment (start 40 67.34) (end 34 67.34) (width 1) (layer "B.Cu") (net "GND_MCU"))
 (segment (start 62.86 21.62) (end 67 21.62) (width 1) (layer "B.Cu") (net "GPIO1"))
 (segment (start 67 21.62) (end 69 20) (width 1) (layer "B.Cu") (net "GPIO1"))
 (segment (start 69 20) (end 73 20) (width 1) (layer "B.Cu") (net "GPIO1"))
 (segment (start 68 24.16) (end 68 30) (width 1) (layer "B.Cu") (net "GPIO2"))
 (segment (start 62.86 24.16) (end 68 24.16) (width 1) (layer "B.Cu") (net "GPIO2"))
 (segment (start 68 30) (end 69 30) (width 1) (layer "B.Cu") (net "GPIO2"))
 (segment (start 69 30) (end 73 30) (width 1) (layer "B.Cu") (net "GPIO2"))
 (segment (start 89 50.16) (end 94.08 50.16) (width 1) (layer "B.Cu") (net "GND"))
 (segment (start 73 40) (end 73 36.8) (width 1) (layer "B.Cu") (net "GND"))
 (segment (start 73 36.8) (end 94.08 36.8) (width 1) (layer "B.Cu") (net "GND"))
 (segment (start 14 24) (end 8 24) (width 1) (layer "B.Cu") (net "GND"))
 (segment (start 15 83) (end 8 83) (width 1) (layer "B.Cu") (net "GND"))
 (segment (start 8 19.08) (end 8 93) (width 2) (layer "B.Cu") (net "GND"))
 (segment (start 8 93) (end 94.08 93) (width 2) (layer "B.Cu") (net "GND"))
 (segment (start 40.4 82) (end 40.4 93) (width 1) (layer "B.Cu") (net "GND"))
 (segment (start 94.08 93) (end 94.08 20) (width 2) (layer "B.Cu") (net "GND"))
 (segment (start 8.92 34) (end 8 34) (width 1) (layer "B.Cu") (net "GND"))
 (segment (start 13.08 89) (end 20 89) (width 1.5) (layer "B.Cu") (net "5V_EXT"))
 (segment (start 13.08 39) (end 13.08 75) (width 1.5) (layer "B.Cu") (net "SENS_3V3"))
 (segment (start 13.08 79.5) (end 20.08 79.5) (width 1.5) (layer "B.Cu") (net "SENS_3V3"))
 (segment (start 20.08 79.5) (end 20.08 83) (width 1.5) (layer "B.Cu") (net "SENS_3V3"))
 (segment (start 13.08 75) (end 13.08 79.5) (width 1.5) (layer "B.Cu") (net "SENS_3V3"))
 (segment (start 18.16 39) (end 18.16 75) (width 1) (layer "B.Cu") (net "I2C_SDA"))
 (segment (start 23.24 39) (end 23.24 75) (width 1) (layer "B.Cu") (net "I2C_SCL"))
 (segment (start 8 14) (end 14 14) (width 1) (layer "B.Cu") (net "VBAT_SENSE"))
 (segment (start 24.16 14) (end 24.16 29) (width 1) (layer "B.Cu") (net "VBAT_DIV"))
 (segment (start 14 34) (end 18.16 34) (width 1) (layer "B.Cu") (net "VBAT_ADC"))
 (segment (start 14 29) (end 14 34) (width 1) (layer "B.Cu") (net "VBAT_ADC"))
 (segment (start 69 60) (end 73 60) (width 1) (layer "B.Cu") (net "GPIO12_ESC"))
 (segment (start 83.16 60) (end 89 60) (width 1) (layer "B.Cu") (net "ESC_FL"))
 (segment (start 83.16 20) (end 89 20) (width 1) (layer "B.Cu") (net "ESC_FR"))
 (segment (start 83.16 30) (end 89 30) (width 1) (layer "B.Cu") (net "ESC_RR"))
 (segment (start 69 70) (end 73 70) (width 1) (layer "B.Cu") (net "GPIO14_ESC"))
 (segment (start 83.16 70) (end 89 70) (width 1) (layer "B.Cu") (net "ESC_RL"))
 (segment (start 78 40) (end 89 40) (width 1) (layer "B.Cu") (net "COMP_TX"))
 (segment (start 78 45.08) (end 89 45.08) (width 1) (layer "B.Cu") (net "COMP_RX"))
 (segment (start 68 50.16) (end 73 50.16) (width 1) (layer "B.Cu") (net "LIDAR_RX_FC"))
 (segment (start 68 55.24) (end 73 55.24) (width 1) (layer "B.Cu") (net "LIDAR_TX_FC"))
 (segment (start 25.16 83) (end 25.16 88) (width 1) (layer "B.Cu") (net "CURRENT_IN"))
 (segment (start 35.32 88) (end 35.32 77) (width 1) (layer "B.Cu") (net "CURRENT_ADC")))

